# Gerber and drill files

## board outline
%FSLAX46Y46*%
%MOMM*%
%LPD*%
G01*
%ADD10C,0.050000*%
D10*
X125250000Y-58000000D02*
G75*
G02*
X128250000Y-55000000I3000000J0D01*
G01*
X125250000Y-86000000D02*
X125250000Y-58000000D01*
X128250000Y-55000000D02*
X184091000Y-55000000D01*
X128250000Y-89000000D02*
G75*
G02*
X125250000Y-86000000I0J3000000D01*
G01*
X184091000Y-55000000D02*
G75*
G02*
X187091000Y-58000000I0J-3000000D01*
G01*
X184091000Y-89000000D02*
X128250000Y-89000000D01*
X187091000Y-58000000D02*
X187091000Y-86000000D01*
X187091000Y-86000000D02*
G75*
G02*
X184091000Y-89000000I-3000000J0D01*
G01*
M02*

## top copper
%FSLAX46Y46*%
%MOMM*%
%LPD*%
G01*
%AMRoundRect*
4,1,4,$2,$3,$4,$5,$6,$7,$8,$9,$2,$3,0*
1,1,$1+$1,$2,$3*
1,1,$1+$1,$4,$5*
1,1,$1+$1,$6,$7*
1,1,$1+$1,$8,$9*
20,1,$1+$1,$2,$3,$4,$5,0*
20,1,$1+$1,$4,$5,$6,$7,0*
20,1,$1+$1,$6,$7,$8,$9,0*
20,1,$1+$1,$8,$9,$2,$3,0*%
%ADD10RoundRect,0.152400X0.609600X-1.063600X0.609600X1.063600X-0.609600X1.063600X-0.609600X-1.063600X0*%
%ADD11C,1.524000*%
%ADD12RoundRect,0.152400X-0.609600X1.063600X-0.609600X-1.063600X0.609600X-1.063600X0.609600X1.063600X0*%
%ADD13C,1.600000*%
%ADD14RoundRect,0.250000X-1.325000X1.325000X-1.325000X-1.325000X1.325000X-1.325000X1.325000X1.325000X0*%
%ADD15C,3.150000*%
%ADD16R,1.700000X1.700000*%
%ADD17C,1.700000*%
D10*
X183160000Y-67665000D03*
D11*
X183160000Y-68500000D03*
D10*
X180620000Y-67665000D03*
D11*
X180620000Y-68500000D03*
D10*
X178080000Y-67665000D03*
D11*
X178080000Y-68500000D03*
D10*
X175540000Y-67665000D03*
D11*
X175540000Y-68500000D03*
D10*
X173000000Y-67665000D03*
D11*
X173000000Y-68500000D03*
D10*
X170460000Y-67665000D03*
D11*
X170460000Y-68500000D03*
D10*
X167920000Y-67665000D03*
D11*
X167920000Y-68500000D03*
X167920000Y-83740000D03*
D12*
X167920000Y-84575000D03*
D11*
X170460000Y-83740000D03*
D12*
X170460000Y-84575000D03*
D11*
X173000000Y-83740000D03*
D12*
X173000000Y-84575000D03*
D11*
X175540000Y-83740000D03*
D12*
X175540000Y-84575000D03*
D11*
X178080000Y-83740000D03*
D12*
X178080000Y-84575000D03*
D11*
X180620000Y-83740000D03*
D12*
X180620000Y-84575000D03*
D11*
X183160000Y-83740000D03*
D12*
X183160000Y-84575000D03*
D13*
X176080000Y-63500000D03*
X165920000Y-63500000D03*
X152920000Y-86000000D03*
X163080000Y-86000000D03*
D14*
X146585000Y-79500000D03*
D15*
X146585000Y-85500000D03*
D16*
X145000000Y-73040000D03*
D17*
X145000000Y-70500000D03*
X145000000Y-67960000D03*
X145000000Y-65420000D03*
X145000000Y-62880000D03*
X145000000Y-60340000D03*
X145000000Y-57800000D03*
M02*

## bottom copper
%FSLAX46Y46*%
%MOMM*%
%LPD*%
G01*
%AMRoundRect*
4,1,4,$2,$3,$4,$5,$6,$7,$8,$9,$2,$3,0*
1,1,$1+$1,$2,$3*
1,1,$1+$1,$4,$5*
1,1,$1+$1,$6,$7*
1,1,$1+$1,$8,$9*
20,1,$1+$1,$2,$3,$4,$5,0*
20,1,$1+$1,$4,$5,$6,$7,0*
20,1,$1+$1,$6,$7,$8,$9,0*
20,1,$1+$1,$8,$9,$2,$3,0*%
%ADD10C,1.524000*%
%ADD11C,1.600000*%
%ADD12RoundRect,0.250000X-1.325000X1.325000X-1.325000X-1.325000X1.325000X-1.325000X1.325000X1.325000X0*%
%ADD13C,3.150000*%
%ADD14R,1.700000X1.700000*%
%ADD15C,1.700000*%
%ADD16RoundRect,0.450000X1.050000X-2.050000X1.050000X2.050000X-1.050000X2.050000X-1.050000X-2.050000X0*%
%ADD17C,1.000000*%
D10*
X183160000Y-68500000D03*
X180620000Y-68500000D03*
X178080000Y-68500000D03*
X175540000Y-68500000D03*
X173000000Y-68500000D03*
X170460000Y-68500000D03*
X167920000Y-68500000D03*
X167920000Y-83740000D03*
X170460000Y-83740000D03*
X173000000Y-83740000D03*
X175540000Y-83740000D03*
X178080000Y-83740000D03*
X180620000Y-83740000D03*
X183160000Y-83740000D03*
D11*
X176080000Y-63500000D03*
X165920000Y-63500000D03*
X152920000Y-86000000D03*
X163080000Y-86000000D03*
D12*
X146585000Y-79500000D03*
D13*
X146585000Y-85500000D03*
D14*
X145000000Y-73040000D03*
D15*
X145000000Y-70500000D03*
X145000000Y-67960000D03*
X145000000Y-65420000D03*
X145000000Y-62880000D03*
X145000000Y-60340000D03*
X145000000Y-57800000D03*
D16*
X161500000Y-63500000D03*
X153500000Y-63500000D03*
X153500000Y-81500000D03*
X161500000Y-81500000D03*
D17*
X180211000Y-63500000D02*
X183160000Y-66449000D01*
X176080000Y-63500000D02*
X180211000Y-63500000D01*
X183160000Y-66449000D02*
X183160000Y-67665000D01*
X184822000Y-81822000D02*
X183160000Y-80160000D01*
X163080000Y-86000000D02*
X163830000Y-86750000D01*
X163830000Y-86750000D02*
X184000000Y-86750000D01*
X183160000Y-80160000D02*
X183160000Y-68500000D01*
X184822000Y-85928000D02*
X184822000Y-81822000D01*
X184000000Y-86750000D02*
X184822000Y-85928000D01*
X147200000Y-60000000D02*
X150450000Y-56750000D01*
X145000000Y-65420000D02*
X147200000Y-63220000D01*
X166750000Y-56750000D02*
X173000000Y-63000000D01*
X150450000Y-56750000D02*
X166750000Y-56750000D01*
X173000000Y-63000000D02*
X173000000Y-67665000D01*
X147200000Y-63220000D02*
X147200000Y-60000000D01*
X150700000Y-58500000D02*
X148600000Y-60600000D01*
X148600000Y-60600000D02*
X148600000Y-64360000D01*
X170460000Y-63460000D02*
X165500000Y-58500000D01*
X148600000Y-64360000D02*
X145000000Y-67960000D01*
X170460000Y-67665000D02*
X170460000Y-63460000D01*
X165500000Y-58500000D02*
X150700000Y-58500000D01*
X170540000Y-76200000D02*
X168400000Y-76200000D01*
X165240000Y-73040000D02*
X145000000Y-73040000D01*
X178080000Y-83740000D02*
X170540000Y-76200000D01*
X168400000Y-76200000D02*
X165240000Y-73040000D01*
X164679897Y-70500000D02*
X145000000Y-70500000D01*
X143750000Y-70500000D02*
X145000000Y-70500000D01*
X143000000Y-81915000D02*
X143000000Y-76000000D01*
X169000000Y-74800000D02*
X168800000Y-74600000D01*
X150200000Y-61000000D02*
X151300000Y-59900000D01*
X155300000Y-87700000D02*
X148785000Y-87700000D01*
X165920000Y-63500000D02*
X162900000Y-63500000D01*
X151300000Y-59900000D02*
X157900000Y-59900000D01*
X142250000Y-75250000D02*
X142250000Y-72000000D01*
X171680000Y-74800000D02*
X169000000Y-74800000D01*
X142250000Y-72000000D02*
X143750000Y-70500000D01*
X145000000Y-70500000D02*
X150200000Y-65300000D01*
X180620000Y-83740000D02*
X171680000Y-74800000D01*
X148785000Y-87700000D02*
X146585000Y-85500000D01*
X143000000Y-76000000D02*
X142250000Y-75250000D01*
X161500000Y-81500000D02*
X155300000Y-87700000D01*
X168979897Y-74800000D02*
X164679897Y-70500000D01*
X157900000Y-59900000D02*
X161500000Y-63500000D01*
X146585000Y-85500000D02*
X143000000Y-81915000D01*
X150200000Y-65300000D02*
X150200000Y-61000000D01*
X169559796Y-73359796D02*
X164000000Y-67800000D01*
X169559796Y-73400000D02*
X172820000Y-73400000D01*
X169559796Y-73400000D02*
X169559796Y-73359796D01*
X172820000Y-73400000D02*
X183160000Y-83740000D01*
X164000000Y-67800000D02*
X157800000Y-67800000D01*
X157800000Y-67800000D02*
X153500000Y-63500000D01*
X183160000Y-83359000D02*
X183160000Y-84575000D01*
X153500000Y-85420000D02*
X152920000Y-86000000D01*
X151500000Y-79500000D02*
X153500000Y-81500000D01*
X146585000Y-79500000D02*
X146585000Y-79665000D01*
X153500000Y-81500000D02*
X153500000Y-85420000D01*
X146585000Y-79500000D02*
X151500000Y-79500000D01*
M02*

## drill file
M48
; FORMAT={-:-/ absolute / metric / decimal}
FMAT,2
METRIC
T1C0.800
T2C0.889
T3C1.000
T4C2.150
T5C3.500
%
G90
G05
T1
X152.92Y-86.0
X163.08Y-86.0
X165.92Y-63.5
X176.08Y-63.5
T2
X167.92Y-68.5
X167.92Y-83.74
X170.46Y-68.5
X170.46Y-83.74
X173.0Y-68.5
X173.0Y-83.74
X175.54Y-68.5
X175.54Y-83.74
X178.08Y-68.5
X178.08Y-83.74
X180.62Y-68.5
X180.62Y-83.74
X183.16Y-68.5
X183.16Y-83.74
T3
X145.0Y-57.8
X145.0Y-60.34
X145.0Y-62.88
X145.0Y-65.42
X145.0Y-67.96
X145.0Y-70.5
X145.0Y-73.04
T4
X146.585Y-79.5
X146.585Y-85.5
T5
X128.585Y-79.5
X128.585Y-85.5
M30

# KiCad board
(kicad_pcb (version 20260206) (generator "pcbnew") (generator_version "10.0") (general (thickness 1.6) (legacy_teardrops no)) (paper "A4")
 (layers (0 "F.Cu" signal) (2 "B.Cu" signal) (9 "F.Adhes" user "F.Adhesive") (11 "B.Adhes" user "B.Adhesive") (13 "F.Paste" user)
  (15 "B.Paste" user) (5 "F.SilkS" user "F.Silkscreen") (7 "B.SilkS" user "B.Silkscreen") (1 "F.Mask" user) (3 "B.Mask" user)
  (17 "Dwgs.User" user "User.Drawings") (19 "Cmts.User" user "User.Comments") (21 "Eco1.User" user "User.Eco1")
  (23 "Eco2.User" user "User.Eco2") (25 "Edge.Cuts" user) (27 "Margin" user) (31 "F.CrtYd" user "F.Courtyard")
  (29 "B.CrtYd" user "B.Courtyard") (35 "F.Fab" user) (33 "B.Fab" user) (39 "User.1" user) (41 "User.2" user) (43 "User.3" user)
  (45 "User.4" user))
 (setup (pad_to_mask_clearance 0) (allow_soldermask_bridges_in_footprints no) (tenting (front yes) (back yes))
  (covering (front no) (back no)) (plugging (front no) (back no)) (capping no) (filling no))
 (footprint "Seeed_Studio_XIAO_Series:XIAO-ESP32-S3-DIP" (layer "F.Cu") (at 175.54 76.12)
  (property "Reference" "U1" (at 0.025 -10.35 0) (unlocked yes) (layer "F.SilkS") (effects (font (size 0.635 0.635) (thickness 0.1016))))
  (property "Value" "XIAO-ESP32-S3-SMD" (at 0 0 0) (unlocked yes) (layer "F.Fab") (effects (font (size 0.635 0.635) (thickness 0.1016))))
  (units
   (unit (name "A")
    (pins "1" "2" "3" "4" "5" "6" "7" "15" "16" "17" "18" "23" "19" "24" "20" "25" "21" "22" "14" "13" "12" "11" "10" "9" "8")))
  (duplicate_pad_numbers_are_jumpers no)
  (pad "1" smd roundrect (at 7.62 -8.455 90) (size 2.432 1.524) (layers "F.Cu" "F.Mask") (roundrect_rratio 0.1) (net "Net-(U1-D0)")
   (thermal_bridge_angle 45))
  (pad "1" thru_hole circle (at 7.62 -7.62 90) (size 1.524 1.524) (drill 0.889) (layers "*.Cu" "*.Mask") (remove_unused_layers no)
   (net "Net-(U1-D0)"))
  (pad "2" smd roundrect (at 5.08 -8.455 90) (size 2.432 1.524) (layers "F.Cu" "F.Mask") (roundrect_rratio 0.1)
   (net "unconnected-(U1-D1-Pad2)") (thermal_bridge_angle 45))
  (pad "2" thru_hole circle (at 5.08 -7.62 90) (size 1.524 1.524) (drill 0.889) (layers "*.Cu" "*.Mask") (remove_unused_layers no)
   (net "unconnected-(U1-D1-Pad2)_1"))
  (pad "3" smd roundrect (at 2.54 -8.455 90) (size 2.432 1.524) (layers "F.Cu" "F.Mask") (roundrect_rratio 0.1)
   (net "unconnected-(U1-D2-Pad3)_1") (thermal_bridge_angle 45))
  (pad "3" thru_hole circle (at 2.54 -7.62 90) (size 1.524 1.524) (drill 0.889) (layers "*.Cu" "*.Mask") (remove_unused_layers no)
   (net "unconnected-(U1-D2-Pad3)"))
  (pad "4" smd roundrect (at 0 -8.455 90) (size 2.432 1.524) (layers "F.Cu" "F.Mask") (roundrect_rratio 0.1)
   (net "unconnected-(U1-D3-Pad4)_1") (thermal_bridge_angle 45))
  (pad "4" thru_hole circle (at 0 -7.62 90) (size 1.524 1.524) (drill 0.889) (layers "*.Cu" "*.Mask") (remove_unused_layers no)
   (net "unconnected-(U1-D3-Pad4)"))
  (pad "5" smd roundrect (at -2.54 -8.455 90) (size 2.432 1.524) (layers "F.Cu" "F.Mask") (roundrect_rratio 0.1) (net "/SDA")
   (thermal_bridge_angle 45))
  (pad "5" thru_hole circle (at -2.54 -7.62 90) (size 1.524 1.524) (drill 0.889) (layers "*.Cu" "*.Mask") (remove_unused_layers no)
   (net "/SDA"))
  (pad "6" smd roundrect (at -5.08 -8.455 90) (size 2.432 1.524) (layers "F.Cu" "F.Mask") (roundrect_rratio 0.1) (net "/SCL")
   (thermal_bridge_angle 45))
  (pad "6" thru_hole circle (at -5.08 -7.62 90) (size 1.524 1.524) (drill 0.889) (layers "*.Cu" "*.Mask") (remove_unused_layers no)
   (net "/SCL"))
  (pad "7" smd roundrect (at -7.62 -8.455 90) (size 2.432 1.524) (layers "F.Cu" "F.Mask") (roundrect_rratio 0.1)
   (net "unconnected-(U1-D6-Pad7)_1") (thermal_bridge_angle 45))
  (pad "7" thru_hole circle (at -7.62 -7.62 90) (size 1.524 1.524) (drill 0.889) (layers "*.Cu" "*.Mask") (remove_unused_layers no)
   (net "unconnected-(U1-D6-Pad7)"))
  (pad "8" thru_hole circle (at -7.62 7.62 270) (size 1.524 1.524) (drill 0.889) (layers "*.Cu" "*.Mask") (remove_unused_layers no)
   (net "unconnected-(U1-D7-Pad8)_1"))
  (pad "8" smd roundrect (at -7.62 8.455 270) (size 2.432 1.524) (layers "F.Cu" "F.Mask") (roundrect_rratio 0.1)
   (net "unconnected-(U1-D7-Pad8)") (thermal_bridge_angle 45))
  (pad "9" thru_hole circle (at -5.08 7.62 270) (size 1.524 1.524) (drill 0.889) (layers "*.Cu" "*.Mask") (remove_unused_layers no)
   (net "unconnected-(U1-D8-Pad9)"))
  (pad "9" smd roundrect (at -5.08 8.455 270) (size 2.432 1.524) (layers "F.Cu" "F.Mask") (roundrect_rratio 0.1)
   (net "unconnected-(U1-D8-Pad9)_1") (thermal_bridge_angle 45))
  (pad "10" thru_hole circle (at -2.54 7.62 270) (size 1.524 1.524) (drill 0.889) (layers "*.Cu" "*.Mask") (remove_unused_layers no)
   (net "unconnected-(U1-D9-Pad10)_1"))
  (pad "10" smd roundrect (at -2.54 8.455 270) (size 2.432 1.524) (layers "F.Cu" "F.Mask") (roundrect_rratio 0.1)
   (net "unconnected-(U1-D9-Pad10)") (thermal_bridge_angle 45))
  (pad "11" thru_hole circle (at 0 7.62 270) (size 1.524 1.524) (drill 0.889) (layers "*.Cu" "*.Mask") (remove_unused_layers no)
   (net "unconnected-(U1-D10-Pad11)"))
  (pad "11" smd roundrect (at 0 8.455 270) (size 2.432 1.524) (layers "F.Cu" "F.Mask") (roundrect_rratio 0.1)
   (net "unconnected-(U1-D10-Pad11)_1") (thermal_bridge_angle 45))
  (pad "12" thru_hole circle (at 2.54 7.62 270) (size 1.524 1.524) (drill 0.889) (layers "*.Cu" "*.Mask") (remove_unused_layers no)
   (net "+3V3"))
  (pad "12" smd roundrect (at 2.54 8.455 270) (size 2.432 1.524) (layers "F.Cu" "F.Mask") (roundrect_rratio 0.1) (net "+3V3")
   (thermal_bridge_angle 45))
  (pad "13" thru_hole circle (at 5.08 7.62 270) (size 1.524 1.524) (drill 0.889) (layers "*.Cu" "*.Mask") (remove_unused_layers no)
   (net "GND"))
  (pad "13" smd roundrect (at 5.08 8.455 270) (size 2.432 1.524) (layers "F.Cu" "F.Mask") (roundrect_rratio 0.1) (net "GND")
   (thermal_bridge_angle 45))
  (pad "14" thru_hole circle (at 7.62 7.62 270) (size 1.524 1.524) (drill 0.889) (layers "*.Cu" "*.Mask") (remove_unused_layers no)
   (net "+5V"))
  (pad "14" smd roundrect (at 7.62 8.455 270) (size 2.432 1.524) (layers "F.Cu" "F.Mask") (roundrect_rratio 0.1) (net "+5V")
   (thermal_bridge_angle 45)))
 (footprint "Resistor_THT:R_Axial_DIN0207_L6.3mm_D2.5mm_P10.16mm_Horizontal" (layer "F.Cu") (at 176.08 63.5 180)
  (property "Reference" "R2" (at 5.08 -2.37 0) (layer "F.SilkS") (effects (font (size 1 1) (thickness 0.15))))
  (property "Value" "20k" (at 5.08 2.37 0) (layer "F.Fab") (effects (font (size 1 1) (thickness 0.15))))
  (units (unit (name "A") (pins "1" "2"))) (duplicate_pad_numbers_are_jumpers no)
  (pad "1" thru_hole circle (at 0 0 180) (size 1.6 1.6) (drill 0.8) (layers "*.Cu" "*.Mask") (remove_unused_layers no) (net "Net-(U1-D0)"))
  (pad "2" thru_hole circle (at 10.16 0 180) (size 1.6 1.6) (drill 0.8) (layers "*.Cu" "*.Mask") (remove_unused_layers no) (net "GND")))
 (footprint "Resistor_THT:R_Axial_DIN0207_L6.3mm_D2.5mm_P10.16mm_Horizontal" (layer "F.Cu") (at 152.92 86)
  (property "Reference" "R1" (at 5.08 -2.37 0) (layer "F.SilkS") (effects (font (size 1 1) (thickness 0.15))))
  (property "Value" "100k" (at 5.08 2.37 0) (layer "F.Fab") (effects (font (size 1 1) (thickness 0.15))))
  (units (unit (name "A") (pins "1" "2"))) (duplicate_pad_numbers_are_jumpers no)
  (pad "1" thru_hole circle (at 0 0) (size 1.6 1.6) (drill 0.8) (layers "*.Cu" "*.Mask") (remove_unused_layers no) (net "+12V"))
  (pad "2" thru_hole circle (at 10.16 0) (size 1.6 1.6) (drill 0.8) (layers "*.Cu" "*.Mask") (remove_unused_layers no) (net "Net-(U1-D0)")))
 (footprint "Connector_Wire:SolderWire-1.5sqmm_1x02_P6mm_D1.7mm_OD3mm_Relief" (layer "F.Cu") (at 146.585 79.5 -90)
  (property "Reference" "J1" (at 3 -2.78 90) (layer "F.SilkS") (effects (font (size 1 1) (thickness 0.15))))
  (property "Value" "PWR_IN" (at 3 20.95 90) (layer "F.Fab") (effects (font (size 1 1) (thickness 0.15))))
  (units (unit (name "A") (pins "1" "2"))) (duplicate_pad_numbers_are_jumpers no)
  (pad "" np_thru_hole circle (at 0 18 270) (size 3.5 3.5) (drill 3.5) (layers "*.Cu" "*.Mask"))
  (pad "" np_thru_hole circle (at 6 18 270) (size 3.5 3.5) (drill 3.5) (layers "*.Cu" "*.Mask"))
  (pad "1" thru_hole roundrect (at 0 0 270) (size 3.15 3.15) (drill 2.15) (layers "*.Cu" "*.Mask") (remove_unused_layers no)
   (roundrect_rratio 0.079365) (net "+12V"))
  (pad "2" thru_hole circle (at 6 0 270) (size 3.15 3.15) (drill 2.15) (layers "*.Cu" "*.Mask") (remove_unused_layers no) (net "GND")))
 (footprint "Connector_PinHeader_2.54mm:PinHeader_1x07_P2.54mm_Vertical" (layer "F.Cu") (at 145 73.04 180)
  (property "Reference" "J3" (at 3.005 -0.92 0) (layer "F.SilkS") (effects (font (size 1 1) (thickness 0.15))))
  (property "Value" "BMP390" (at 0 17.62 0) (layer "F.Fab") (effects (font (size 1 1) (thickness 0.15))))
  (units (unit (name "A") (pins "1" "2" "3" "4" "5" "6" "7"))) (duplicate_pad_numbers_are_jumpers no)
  (pad "1" thru_hole rect (at 0 0 180) (size 1.7 1.7) (drill 1) (layers "*.Cu" "*.Mask") (remove_unused_layers no) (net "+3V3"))
  (pad "2" thru_hole circle (at 0 2.54 180) (size 1.7 1.7) (drill 1) (layers "*.Cu" "*.Mask") (remove_unused_layers no) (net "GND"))
  (pad "3" thru_hole circle (at 0 5.08 180) (size 1.7 1.7) (drill 1) (layers "*.Cu" "*.Mask") (remove_unused_layers no) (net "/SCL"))
  (pad "4" thru_hole circle (at 0 7.62 180) (size 1.7 1.7) (drill 1) (layers "*.Cu" "*.Mask") (remove_unused_layers no) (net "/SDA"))
  (pad "5" thru_hole circle (at 0 10.16 180) (size 1.7 1.7) (drill 1) (layers "*.Cu" "*.Mask") (remove_unused_layers no)
   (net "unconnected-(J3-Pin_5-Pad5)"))
  (pad "6" thru_hole circle (at 0 12.7 180) (size 1.7 1.7) (drill 1) (layers "*.Cu" "*.Mask") (remove_unused_layers no)
   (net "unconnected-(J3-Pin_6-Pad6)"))
  (pad "7" thru_hole circle (at 0 15.24 180) (size 1.7 1.7) (drill 1) (layers "*.Cu" "*.Mask") (remove_unused_layers no)
   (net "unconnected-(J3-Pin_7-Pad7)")))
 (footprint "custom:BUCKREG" (layer "B.Cu") (at 157.5 72.5 90)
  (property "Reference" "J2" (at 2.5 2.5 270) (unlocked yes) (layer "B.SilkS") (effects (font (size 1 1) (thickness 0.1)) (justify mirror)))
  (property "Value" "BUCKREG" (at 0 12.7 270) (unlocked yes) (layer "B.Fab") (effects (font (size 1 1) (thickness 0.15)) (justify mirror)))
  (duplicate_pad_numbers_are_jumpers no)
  (pad "1" smd roundrect (at 9 4 90) (size 5 3) (layers "B.Cu" "B.Mask" "B.Paste") (roundrect_rratio 0.15) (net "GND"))
  (pad "2" smd roundrect (at 9 -4 90) (size 5 3) (layers "B.Cu" "B.Mask" "B.Paste") (roundrect_rratio 0.15) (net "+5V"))
  (pad "3" smd roundrect (at -9 -4 90) (size 5 3) (layers "B.Cu" "B.Mask" "B.Paste") (roundrect_rratio 0.15) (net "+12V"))
  (pad "4" smd roundrect (at -9 4 90) (size 5 3) (layers "B.Cu" "B.Mask" "B.Paste") (roundrect_rratio 0.15) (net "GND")))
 (gr_arc (start 125.25 58) (mid 126.12868 55.87868) (end 128.25 55) (stroke (width 0.05) (type default)) (layer "Edge.Cuts"))
 (gr_line (start 125.25 86) (end 125.25 58) (stroke (width 0.05) (type default)) (layer "Edge.Cuts"))
 (gr_line (start 128.25 55) (end 184.091 55) (stroke (width 0.05) (type default)) (layer "Edge.Cuts"))
 (gr_arc (start 128.25 89) (mid 126.12868 88.12132) (end 125.25 86) (stroke (width 0.05) (type default)) (layer "Edge.Cuts"))
 (gr_arc (start 184.091 55) (mid 186.21232 55.87868) (end 187.091 58) (stroke (width 0.05) (type default)) (layer "Edge.Cuts"))
 (gr_line (start 184.091 89) (end 128.25 89) (stroke (width 0.05) (type default)) (layer "Edge.Cuts"))
 (gr_line (start 187.091 58) (end 187.091 86) (stroke (width 0.05) (type default)) (layer "Edge.Cuts"))
 (gr_arc (start 187.091 86) (mid 186.21232 88.12132) (end 184.091 89) (stroke (width 0.05) (type default)) (layer "Edge.Cuts"))
 (segment (start 180.211 63.5) (end 183.16 66.449) (width 1) (layer "B.Cu") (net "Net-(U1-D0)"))
 (segment (start 176.08 63.5) (end 180.211 63.5) (width 1) (layer "B.Cu") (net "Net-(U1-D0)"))
 (segment (start 183.16 66.449) (end 183.16 67.665) (width 1) (layer "B.Cu") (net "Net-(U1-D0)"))
 (segment (start 184.822 81.822) (end 183.16 80.16) (width 1) (layer "B.Cu") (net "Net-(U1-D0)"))
 (segment (start 163.08 86) (end 163.83 86.75) (width 1) (layer "B.Cu") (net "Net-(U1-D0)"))
 (segment (start 163.83 86.75) (end 184 86.75) (width 1) (layer "B.Cu") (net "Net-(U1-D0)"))
 (segment (start 183.16 80.16) (end 183.16 68.5) (width 1) (layer "B.Cu") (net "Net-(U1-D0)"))
 (segment (start 184.822 85.928) (end 184.822 81.822) (width 1) (layer "B.Cu") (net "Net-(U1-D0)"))
 (segment (start 184 86.75) (end 184.822 85.928) (width 1) (layer "B.Cu") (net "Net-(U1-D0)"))
 (segment (start 147.2 60) (end 150.45 56.75) (width 1) (layer "B.Cu") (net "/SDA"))
 (segment (start 145 65.42) (end 147.2 63.22) (width 1) (layer "B.Cu") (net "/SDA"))
 (segment (start 166.75 56.75) (end 173 63) (width 1) (layer "B.Cu") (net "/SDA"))
 (segment (start 150.45 56.75) (end 166.75 56.75) (width 1) (layer "B.Cu") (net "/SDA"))
 (segment (start 173 63) (end 173 67.665) (width 1) (layer "B.Cu") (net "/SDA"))
 (segment (start 147.2 63.22) (end 147.2 60) (width 1) (layer "B.Cu") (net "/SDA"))
 (segment (start 150.7 58.5) (end 148.6 60.6) (width 1) (layer "B.Cu") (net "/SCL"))
 (segment (start 148.6 60.6) (end 148.6 64.36) (width 1) (layer "B.Cu") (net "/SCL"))
 (segment (start 170.46 63.46) (end 165.5 58.5) (width 1) (layer "B.Cu") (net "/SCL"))
 (segment (start 148.6 64.36) (end 145 67.96) (width 1) (layer "B.Cu") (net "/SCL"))
 (segment (start 170.46 67.665) (end 170.46 63.46) (width 1) (layer "B.Cu") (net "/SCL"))
 (segment (start 165.5 58.5) (end 150.7 58.5) (width 1) (layer "B.Cu") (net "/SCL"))
 (segment (start 170.54 76.2) (end 168.4 76.2) (width 1) (layer "B.Cu") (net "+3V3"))
 (segment (start 165.24 73.04) (end 145 73.04) (width 1) (layer "B.Cu") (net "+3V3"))
 (segment (start 178.08 83.74) (end 170.54 76.2) (width 1) (layer "B.Cu") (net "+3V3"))
 (segment (start 168.4 76.2) (end 165.24 73.04) (width 1) (layer "B.Cu") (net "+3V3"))
 (segment (start 164.679897 70.5) (end 145 70.5) (width 1) (layer "B.Cu") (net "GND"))
 (segment (start 143.75 70.5) (end 145 70.5) (width 1) (layer "B.Cu") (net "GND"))
 (segment (start 143 81.915) (end 143 76) (width 1) (layer "B.Cu") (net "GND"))
 (segment (start 169 74.8) (end 168.8 74.6) (width 1) (layer "B.Cu") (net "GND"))
 (segment (start 150.2 61) (end 151.3 59.9) (width 1) (layer "B.Cu") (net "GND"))
 (segment (start 155.3 87.7) (end 148.785 87.7) (width 1) (layer "B.Cu") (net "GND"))
 (segment (start 165.92 63.5) (end 162.9 63.5) (width 1) (layer "B.Cu") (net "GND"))
 (segment (start 151.3 59.9) (end 157.9 59.9) (width 1) (layer "B.Cu") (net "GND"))
 (segment (start 142.25 75.25) (end 142.25 72) (width 1) (layer "B.Cu") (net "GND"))
 (segment (start 171.68 74.8) (end 169 74.8) (width 1) (layer "B.Cu") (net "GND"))
 (segment (start 142.25 72) (end 143.75 70.5) (width 1) (layer "B.Cu") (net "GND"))
 (segment (start 145 70.5) (end 150.2 65.3) (width 1) (layer "B.Cu") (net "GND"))
 (segment (start 180.62 83.74) (end 171.68 74.8) (width 1) (layer "B.Cu") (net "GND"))
 (segment (start 148.785 87.7) (end 146.585 85.5) (width 1) (layer "B.Cu") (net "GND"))
 (segment (start 143 76) (end 142.25 75.25) (width 1) (layer "B.Cu") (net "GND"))
 (segment (start 161.5 81.5) (end 155.3 87.7) (width 1) (layer "B.Cu") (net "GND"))
 (segment (start 168.979897 74.8) (end 164.679897 70.5) (width 1) (layer "B.Cu") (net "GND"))
 (segment (start 157.9 59.9) (end 161.5 63.5) (width 1) (layer "B.Cu") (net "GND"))
 (segment (start 146.585 85.5) (end 143 81.915) (width 1) (layer "B.Cu") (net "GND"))
 (segment (start 150.2 65.3) (end 150.2 61) (width 1) (layer "B.Cu") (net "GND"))
 (segment (start 169.559796 73.359796) (end 164 67.8) (width 1) (layer "B.Cu") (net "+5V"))
 (segment (start 169.559796 73.4) (end 172.82 73.4) (width 1) (layer "B.Cu") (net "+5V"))
 (segment (start 169.559796 73.4) (end 169.559796 73.359796) (width 1) (layer "B.Cu") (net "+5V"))
 (segment (start 172.82 73.4) (end 183.16 83.74) (width 1) (layer "B.Cu") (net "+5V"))
 (segment (start 164 67.8) (end 157.8 67.8) (width 1) (layer "B.Cu") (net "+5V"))
 (segment (start 157.8 67.8) (end 153.5 63.5) (width 1) (layer "B.Cu") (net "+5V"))
 (segment (start 183.16 83.359) (end 183.16 84.575) (width 1) (layer "B.Cu") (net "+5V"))
 (segment (start 153.5 85.42) (end 152.92 86) (width 1) (layer "B.Cu") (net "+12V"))
 (segment (start 151.5 79.5) (end 153.5 81.5) (width 1) (layer "B.Cu") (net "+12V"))
 (segment (start 146.585 79.5) (end 146.585 79.665) (width 1) (layer "B.Cu") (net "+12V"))
 (segment (start 153.5 81.5) (end 153.5 85.42) (width 1) (layer "B.Cu") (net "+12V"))
 (segment (start 146.585 79.5) (end 151.5 79.5) (width 1) (layer "B.Cu") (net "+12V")))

